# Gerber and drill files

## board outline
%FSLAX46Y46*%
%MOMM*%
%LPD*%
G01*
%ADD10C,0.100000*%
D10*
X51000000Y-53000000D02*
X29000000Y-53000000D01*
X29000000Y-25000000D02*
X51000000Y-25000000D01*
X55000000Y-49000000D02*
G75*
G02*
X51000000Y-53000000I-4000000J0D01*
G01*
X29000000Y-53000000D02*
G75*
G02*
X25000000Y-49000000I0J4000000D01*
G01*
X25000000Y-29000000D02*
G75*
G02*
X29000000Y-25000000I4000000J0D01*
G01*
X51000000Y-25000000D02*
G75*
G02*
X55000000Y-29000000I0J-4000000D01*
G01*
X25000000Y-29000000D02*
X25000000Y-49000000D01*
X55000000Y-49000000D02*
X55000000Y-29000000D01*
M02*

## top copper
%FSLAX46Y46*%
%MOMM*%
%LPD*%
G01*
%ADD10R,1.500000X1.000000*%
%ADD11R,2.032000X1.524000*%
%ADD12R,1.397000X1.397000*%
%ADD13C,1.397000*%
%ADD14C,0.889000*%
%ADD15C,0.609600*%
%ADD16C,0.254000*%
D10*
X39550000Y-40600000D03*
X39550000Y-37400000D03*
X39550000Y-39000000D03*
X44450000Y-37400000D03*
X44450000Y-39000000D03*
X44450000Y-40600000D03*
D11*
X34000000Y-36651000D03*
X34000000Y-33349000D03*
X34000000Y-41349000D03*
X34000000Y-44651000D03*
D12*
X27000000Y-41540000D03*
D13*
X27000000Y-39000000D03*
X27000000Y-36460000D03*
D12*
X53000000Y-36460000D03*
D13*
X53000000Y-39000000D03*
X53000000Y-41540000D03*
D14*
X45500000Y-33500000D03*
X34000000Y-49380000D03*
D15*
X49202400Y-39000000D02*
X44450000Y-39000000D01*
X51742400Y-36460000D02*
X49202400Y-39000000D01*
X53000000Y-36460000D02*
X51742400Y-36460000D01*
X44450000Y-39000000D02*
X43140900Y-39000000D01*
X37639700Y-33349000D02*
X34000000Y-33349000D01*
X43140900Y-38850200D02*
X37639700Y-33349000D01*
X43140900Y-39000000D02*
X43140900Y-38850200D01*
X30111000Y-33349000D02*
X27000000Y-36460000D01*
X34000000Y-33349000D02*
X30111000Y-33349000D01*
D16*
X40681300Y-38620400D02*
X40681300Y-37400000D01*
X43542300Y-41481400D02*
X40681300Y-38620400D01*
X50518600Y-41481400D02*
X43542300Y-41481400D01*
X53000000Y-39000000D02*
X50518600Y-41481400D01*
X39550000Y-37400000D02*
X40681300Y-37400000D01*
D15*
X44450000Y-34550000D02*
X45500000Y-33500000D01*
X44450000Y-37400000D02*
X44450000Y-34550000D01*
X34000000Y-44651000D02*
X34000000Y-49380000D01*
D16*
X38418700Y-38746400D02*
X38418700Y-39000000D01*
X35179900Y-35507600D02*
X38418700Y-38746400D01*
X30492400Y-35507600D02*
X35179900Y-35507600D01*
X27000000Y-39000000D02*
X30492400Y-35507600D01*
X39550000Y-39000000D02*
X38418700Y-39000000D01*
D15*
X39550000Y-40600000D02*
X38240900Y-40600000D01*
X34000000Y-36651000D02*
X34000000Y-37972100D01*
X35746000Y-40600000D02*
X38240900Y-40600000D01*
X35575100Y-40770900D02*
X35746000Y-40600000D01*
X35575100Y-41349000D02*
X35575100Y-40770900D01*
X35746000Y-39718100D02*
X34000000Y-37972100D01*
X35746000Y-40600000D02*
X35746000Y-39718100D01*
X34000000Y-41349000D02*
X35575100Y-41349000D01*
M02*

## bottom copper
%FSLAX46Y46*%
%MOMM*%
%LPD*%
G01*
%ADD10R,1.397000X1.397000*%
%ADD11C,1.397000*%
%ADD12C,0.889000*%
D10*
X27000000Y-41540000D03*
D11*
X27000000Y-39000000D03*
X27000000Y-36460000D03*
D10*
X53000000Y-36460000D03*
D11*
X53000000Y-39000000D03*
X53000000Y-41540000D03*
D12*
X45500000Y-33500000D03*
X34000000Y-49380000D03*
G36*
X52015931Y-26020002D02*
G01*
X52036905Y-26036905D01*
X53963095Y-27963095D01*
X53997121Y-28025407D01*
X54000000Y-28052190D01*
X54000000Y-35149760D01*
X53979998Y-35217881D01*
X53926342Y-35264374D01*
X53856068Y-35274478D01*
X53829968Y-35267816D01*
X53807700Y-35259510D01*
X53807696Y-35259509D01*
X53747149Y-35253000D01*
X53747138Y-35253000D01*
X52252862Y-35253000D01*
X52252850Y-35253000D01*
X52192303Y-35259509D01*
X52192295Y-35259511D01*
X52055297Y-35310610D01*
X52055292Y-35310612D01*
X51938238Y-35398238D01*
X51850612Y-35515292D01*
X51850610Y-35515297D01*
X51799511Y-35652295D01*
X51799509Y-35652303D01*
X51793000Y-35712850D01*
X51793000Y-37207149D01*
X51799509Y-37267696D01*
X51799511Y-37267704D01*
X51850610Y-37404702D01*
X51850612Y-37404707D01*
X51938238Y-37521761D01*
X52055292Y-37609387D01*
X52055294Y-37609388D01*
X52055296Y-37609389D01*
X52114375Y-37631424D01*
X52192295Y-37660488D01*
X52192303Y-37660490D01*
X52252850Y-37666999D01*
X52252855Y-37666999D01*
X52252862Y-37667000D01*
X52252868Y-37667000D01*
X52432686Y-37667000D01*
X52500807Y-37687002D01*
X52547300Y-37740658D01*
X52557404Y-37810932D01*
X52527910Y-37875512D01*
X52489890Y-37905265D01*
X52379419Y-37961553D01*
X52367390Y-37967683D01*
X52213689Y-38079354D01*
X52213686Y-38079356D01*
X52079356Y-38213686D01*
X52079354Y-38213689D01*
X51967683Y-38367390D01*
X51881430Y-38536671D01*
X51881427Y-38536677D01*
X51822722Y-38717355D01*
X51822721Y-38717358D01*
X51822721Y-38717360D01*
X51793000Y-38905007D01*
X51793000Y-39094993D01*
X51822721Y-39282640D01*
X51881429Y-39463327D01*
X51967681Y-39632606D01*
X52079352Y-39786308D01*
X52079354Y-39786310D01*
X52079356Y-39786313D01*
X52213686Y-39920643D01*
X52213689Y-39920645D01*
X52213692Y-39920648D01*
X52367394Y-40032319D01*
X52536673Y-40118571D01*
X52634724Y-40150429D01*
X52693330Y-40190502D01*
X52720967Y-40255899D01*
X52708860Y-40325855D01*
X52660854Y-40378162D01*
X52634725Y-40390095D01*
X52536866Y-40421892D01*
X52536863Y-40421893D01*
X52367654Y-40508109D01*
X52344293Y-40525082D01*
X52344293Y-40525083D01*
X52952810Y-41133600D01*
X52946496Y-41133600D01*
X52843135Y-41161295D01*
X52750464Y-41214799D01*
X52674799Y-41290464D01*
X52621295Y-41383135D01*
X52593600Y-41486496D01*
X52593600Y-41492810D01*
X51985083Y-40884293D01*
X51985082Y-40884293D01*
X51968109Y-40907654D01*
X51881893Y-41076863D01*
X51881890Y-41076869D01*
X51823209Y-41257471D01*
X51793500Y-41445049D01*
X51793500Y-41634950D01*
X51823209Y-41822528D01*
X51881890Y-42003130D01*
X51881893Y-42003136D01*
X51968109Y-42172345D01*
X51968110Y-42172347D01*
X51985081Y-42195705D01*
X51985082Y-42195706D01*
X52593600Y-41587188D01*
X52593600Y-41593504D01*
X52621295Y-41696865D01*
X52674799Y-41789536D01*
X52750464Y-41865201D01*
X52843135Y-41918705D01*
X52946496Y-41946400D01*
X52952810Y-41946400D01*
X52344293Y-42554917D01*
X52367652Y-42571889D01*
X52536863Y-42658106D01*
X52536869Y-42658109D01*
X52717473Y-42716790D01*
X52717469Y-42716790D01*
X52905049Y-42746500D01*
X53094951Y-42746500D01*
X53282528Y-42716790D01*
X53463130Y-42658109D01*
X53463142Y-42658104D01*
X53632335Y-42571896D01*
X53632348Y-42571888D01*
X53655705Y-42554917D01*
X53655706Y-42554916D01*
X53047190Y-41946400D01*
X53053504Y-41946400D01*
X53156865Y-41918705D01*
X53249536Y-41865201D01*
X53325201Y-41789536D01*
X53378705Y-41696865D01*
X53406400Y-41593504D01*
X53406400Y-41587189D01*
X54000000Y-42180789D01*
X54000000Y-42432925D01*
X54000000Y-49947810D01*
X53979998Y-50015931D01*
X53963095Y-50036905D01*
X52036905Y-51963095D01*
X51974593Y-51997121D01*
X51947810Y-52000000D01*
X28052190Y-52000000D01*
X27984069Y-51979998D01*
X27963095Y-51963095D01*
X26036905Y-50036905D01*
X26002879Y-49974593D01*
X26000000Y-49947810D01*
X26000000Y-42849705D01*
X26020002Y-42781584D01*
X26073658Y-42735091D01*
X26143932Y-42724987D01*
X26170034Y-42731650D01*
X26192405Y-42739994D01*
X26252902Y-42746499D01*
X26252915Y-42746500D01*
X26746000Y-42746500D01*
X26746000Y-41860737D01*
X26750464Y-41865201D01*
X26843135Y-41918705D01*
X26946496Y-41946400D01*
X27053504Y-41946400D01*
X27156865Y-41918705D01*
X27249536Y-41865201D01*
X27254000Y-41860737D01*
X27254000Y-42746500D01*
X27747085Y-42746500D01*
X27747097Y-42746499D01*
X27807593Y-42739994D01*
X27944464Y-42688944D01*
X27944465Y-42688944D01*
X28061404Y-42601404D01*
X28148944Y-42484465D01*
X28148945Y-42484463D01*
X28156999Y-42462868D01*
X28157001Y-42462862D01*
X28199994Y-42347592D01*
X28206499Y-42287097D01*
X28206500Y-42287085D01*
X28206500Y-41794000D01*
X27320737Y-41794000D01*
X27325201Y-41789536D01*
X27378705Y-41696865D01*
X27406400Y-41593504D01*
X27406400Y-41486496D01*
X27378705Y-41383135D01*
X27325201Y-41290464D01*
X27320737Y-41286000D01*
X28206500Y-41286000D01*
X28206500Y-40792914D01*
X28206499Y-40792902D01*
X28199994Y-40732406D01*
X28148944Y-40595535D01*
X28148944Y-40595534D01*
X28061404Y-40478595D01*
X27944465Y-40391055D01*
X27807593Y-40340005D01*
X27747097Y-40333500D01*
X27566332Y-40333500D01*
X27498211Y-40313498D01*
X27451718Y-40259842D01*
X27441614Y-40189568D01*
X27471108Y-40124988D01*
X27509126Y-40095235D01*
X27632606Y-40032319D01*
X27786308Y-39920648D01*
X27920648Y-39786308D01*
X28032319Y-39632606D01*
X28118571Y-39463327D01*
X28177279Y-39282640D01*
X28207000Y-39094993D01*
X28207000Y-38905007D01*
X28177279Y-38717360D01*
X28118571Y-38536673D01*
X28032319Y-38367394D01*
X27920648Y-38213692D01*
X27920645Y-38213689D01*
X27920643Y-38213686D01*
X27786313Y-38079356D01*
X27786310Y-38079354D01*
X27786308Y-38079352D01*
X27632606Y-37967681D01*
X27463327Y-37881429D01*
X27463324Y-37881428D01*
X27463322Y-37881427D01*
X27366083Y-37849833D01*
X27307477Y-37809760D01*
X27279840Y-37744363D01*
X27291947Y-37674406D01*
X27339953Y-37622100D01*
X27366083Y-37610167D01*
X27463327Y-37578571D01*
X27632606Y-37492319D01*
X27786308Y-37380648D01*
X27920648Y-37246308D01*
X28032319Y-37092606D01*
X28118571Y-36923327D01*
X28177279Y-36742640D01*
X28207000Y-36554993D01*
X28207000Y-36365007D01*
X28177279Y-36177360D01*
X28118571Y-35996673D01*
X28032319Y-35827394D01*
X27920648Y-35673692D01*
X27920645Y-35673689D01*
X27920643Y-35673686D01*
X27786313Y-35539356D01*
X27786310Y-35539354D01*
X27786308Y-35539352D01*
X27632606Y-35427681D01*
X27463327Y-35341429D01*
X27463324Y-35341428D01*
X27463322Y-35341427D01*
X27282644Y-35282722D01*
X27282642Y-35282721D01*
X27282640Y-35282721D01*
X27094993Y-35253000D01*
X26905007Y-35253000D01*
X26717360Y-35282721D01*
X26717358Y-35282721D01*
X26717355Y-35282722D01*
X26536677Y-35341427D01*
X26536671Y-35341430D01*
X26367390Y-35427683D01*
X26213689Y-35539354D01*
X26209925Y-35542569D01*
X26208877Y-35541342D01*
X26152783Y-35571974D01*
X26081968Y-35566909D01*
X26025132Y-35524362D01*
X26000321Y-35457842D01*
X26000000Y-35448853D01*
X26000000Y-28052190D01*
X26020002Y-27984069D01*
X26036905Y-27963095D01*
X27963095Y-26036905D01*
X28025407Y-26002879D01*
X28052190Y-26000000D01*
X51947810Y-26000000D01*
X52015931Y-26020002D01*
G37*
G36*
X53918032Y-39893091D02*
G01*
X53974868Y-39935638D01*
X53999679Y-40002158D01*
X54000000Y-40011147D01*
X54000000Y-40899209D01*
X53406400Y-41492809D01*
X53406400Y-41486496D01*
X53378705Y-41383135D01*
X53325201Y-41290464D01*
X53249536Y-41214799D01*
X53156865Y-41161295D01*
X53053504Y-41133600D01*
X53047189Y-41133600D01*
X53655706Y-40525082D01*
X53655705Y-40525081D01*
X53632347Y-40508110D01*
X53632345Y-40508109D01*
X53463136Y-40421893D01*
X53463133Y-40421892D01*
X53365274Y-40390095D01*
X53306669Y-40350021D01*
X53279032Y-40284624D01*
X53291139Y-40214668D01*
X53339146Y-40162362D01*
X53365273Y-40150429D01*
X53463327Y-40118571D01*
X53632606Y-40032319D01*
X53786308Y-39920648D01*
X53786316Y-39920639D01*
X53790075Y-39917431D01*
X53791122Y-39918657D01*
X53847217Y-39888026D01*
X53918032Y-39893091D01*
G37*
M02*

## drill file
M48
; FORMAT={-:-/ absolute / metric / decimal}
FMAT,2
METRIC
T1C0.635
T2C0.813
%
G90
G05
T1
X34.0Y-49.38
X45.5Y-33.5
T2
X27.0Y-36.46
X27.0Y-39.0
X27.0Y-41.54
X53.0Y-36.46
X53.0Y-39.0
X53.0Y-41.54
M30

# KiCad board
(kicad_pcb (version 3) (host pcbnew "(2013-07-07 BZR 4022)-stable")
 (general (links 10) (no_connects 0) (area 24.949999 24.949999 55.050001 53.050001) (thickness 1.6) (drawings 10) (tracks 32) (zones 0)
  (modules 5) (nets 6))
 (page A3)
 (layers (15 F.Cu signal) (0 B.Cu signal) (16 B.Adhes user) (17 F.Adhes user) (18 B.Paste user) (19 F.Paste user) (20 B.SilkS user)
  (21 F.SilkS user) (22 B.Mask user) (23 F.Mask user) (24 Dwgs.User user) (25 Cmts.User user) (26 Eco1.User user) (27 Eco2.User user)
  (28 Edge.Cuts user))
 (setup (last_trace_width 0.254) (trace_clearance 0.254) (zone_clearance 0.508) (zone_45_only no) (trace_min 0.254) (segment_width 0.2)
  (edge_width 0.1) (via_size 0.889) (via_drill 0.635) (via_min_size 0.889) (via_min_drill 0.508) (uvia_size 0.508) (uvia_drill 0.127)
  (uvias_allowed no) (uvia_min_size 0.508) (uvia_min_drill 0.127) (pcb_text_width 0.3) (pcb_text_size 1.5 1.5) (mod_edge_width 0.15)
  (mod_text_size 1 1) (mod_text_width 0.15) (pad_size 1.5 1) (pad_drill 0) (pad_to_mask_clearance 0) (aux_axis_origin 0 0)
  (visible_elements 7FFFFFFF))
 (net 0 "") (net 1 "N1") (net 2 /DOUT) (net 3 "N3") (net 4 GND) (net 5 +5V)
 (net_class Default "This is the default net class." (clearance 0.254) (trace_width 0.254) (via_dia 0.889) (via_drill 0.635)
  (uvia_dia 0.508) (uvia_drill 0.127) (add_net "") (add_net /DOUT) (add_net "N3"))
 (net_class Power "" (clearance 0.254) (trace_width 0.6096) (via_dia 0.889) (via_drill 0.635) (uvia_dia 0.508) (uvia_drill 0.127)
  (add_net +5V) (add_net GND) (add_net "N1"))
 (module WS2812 (layer F.Cu) (at 42 39)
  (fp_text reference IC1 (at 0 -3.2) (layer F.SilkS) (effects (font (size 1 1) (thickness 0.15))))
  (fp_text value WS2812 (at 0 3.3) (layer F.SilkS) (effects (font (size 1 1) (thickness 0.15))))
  (pad 3 smd rect (at -2.45 1.6) (size 1.5 1) (layers F.Cu F.Paste F.Mask) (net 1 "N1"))
  (pad 1 smd rect (at -2.45 -1.6) (size 1.5 1) (layers F.Cu F.Paste F.Mask) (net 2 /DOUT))
  (pad 2 smd rect (at -2.45 0) (size 1.5 1) (layers F.Cu F.Paste F.Mask) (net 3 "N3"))
  (pad 6 smd rect (at 2.45 -1.6) (size 1.5 1) (layers F.Cu F.Paste F.Mask) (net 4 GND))
  (pad 5 smd rect (at 2.45 0) (size 1.5 1) (layers F.Cu F.Paste F.Mask) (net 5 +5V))
  (pad 4 smd rect (at 1.7 1.1) (size 1.5 1) (drill (offset 0.75 0.5)) (layers F.Cu F.Paste F.Mask)))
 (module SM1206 (layer F.Cu) (at 34 35 90)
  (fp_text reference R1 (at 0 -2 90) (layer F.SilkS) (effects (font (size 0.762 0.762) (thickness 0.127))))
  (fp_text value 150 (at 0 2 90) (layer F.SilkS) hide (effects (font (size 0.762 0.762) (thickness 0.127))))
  (pad 1 smd rect (at -1.651 0 90) (size 1.524 2.032) (layers F.Cu F.Paste F.Mask) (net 1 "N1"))
  (pad 2 smd rect (at 1.651 0 90) (size 1.524 2.032) (layers F.Cu F.Paste F.Mask) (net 5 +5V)))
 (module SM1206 (layer F.Cu) (at 34 43 270)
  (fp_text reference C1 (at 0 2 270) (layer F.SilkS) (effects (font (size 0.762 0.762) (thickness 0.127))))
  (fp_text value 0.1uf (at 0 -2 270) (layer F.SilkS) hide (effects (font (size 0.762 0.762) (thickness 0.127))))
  (pad 1 smd rect (at -1.651 0 270) (size 1.524 2.032) (layers F.Cu F.Paste F.Mask) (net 1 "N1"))
  (pad 2 smd rect (at 1.651 0 270) (size 1.524 2.032) (layers F.Cu F.Paste F.Mask) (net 4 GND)))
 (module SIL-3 (layer F.Cu) (at 27 39 90)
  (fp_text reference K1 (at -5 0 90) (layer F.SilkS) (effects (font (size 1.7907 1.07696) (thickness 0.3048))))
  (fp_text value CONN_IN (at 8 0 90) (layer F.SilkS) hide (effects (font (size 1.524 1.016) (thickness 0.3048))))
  (pad 1 thru_hole rect (at -2.54 0 90) (size 1.397 1.397) (drill 0.8128) (layers *.Cu *.Mask F.SilkS) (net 4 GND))
  (pad 2 thru_hole circle (at 0 0 90) (size 1.397 1.397) (drill 0.8128) (layers *.Cu *.Mask F.SilkS) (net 3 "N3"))
  (pad 3 thru_hole circle (at 2.54 0 90) (size 1.397 1.397) (drill 0.8128) (layers *.Cu *.Mask F.SilkS) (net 5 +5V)))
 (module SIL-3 (layer F.Cu) (at 53 39 270)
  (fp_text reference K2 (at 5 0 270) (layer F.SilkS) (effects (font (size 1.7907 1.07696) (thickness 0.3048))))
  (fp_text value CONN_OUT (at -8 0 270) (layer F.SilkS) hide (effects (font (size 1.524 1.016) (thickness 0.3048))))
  (pad 1 thru_hole rect (at -2.54 0 270) (size 1.397 1.397) (drill 0.8128) (layers *.Cu *.Mask F.SilkS) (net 5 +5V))
  (pad 2 thru_hole circle (at 0 0 270) (size 1.397 1.397) (drill 0.8128) (layers *.Cu *.Mask F.SilkS) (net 2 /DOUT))
  (pad 3 thru_hole circle (at 2.54 0 270) (size 1.397 1.397) (drill 0.8128) (layers *.Cu *.Mask F.SilkS) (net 4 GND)))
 (gr_line (start 51 53) (end 29 53) (angle 90) (layer Edge.Cuts) (width 0.1))
 (gr_line (start 29 25) (end 51 25) (angle 90) (layer Edge.Cuts) (width 0.1))
 (gr_arc (start 51 49) (end 55 49) (angle 90) (layer Edge.Cuts) (width 0.1))
 (gr_arc (start 29 49) (end 29 53) (angle 90) (layer Edge.Cuts) (width 0.1))
 (gr_arc (start 29 29) (end 25 29) (angle 90) (layer Edge.Cuts) (width 0.1))
 (gr_arc (start 51 29) (end 51 25) (angle 90) (layer Edge.Cuts) (width 0.1))
 (gr_line (start 25 29) (end 25 49) (angle 90) (layer Edge.Cuts) (width 0.1))
 (gr_line (start 55 49) (end 55 29) (angle 90) (layer Edge.Cuts) (width 0.1))
 (segment (start 49.2024 39) (end 44.45 39) (width 0.6096) (layer F.Cu) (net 5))
 (segment (start 51.7424 36.46) (end 49.2024 39) (width 0.6096) (layer F.Cu) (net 5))
 (segment (start 53 36.46) (end 51.7424 36.46) (width 0.6096) (layer F.Cu) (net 5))
 (segment (start 44.45 39) (end 43.1409 39) (width 0.6096) (layer F.Cu) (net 5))
 (segment (start 37.6397 33.349) (end 34 33.349) (width 0.6096) (layer F.Cu) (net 5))
 (segment (start 43.1409 38.8502) (end 37.6397 33.349) (width 0.6096) (layer F.Cu) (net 5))
 (segment (start 43.1409 39) (end 43.1409 38.8502) (width 0.6096) (layer F.Cu) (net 5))
 (segment (start 30.111 33.349) (end 27 36.46) (width 0.6096) (layer F.Cu) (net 5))
 (segment (start 34 33.349) (end 30.111 33.349) (width 0.6096) (layer F.Cu) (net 5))
 (segment (start 40.6813 38.6204) (end 40.6813 37.4) (width 0.254) (layer F.Cu) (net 2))
 (segment (start 43.5423 41.4814) (end 40.6813 38.6204) (width 0.254) (layer F.Cu) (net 2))
 (segment (start 50.5186 41.4814) (end 43.5423 41.4814) (width 0.254) (layer F.Cu) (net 2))
 (segment (start 53 39) (end 50.5186 41.4814) (width 0.254) (layer F.Cu) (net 2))
 (segment (start 39.55 37.4) (end 40.6813 37.4) (width 0.254) (layer F.Cu) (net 2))
 (via (at 45.5 33.5) (size 0.889) (layers F.Cu B.Cu) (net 4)) (via (at 34 49.38) (size 0.889) (layers F.Cu B.Cu) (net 4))
 (segment (start 44.45 34.55) (end 45.5 33.5) (width 0.6096) (layer F.Cu) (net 4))
 (segment (start 44.45 37.4) (end 44.45 34.55) (width 0.6096) (layer F.Cu) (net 4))
 (segment (start 34 44.651) (end 34 49.38) (width 0.6096) (layer F.Cu) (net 4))
 (segment (start 38.4187 38.7464) (end 38.4187 39) (width 0.254) (layer F.Cu) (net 3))
 (segment (start 35.1799 35.5076) (end 38.4187 38.7464) (width 0.254) (layer F.Cu) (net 3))
 (segment (start 30.4924 35.5076) (end 35.1799 35.5076) (width 0.254) (layer F.Cu) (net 3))
 (segment (start 27 39) (end 30.4924 35.5076) (width 0.254) (layer F.Cu) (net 3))
 (segment (start 39.55 39) (end 38.4187 39) (width 0.254) (layer F.Cu) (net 3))
 (segment (start 39.55 40.6) (end 38.2409 40.6) (width 0.6096) (layer F.Cu) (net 1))
 (segment (start 34 36.651) (end 34 37.9721) (width 0.6096) (layer F.Cu) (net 1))
 (segment (start 35.746 40.6) (end 38.2409 40.6) (width 0.6096) (layer F.Cu) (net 1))
 (segment (start 35.5751 40.7709) (end 35.746 40.6) (width 0.6096) (layer F.Cu) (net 1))
 (segment (start 35.5751 41.349) (end 35.5751 40.7709) (width 0.6096) (layer F.Cu) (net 1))
 (segment (start 35.746 39.7181) (end 34 37.9721) (width 0.6096) (layer F.Cu) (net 1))
 (segment (start 35.746 40.6) (end 35.746 39.7181) (width 0.6096) (layer F.Cu) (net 1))
 (segment (start 34 41.349) (end 35.5751 41.349) (width 0.6096) (layer F.Cu) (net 1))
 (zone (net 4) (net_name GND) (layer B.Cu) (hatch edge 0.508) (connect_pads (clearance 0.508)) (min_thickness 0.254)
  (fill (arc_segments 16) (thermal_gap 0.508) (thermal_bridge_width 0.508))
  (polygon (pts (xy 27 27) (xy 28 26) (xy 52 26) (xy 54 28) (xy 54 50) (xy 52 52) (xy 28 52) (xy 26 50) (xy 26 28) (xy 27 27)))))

